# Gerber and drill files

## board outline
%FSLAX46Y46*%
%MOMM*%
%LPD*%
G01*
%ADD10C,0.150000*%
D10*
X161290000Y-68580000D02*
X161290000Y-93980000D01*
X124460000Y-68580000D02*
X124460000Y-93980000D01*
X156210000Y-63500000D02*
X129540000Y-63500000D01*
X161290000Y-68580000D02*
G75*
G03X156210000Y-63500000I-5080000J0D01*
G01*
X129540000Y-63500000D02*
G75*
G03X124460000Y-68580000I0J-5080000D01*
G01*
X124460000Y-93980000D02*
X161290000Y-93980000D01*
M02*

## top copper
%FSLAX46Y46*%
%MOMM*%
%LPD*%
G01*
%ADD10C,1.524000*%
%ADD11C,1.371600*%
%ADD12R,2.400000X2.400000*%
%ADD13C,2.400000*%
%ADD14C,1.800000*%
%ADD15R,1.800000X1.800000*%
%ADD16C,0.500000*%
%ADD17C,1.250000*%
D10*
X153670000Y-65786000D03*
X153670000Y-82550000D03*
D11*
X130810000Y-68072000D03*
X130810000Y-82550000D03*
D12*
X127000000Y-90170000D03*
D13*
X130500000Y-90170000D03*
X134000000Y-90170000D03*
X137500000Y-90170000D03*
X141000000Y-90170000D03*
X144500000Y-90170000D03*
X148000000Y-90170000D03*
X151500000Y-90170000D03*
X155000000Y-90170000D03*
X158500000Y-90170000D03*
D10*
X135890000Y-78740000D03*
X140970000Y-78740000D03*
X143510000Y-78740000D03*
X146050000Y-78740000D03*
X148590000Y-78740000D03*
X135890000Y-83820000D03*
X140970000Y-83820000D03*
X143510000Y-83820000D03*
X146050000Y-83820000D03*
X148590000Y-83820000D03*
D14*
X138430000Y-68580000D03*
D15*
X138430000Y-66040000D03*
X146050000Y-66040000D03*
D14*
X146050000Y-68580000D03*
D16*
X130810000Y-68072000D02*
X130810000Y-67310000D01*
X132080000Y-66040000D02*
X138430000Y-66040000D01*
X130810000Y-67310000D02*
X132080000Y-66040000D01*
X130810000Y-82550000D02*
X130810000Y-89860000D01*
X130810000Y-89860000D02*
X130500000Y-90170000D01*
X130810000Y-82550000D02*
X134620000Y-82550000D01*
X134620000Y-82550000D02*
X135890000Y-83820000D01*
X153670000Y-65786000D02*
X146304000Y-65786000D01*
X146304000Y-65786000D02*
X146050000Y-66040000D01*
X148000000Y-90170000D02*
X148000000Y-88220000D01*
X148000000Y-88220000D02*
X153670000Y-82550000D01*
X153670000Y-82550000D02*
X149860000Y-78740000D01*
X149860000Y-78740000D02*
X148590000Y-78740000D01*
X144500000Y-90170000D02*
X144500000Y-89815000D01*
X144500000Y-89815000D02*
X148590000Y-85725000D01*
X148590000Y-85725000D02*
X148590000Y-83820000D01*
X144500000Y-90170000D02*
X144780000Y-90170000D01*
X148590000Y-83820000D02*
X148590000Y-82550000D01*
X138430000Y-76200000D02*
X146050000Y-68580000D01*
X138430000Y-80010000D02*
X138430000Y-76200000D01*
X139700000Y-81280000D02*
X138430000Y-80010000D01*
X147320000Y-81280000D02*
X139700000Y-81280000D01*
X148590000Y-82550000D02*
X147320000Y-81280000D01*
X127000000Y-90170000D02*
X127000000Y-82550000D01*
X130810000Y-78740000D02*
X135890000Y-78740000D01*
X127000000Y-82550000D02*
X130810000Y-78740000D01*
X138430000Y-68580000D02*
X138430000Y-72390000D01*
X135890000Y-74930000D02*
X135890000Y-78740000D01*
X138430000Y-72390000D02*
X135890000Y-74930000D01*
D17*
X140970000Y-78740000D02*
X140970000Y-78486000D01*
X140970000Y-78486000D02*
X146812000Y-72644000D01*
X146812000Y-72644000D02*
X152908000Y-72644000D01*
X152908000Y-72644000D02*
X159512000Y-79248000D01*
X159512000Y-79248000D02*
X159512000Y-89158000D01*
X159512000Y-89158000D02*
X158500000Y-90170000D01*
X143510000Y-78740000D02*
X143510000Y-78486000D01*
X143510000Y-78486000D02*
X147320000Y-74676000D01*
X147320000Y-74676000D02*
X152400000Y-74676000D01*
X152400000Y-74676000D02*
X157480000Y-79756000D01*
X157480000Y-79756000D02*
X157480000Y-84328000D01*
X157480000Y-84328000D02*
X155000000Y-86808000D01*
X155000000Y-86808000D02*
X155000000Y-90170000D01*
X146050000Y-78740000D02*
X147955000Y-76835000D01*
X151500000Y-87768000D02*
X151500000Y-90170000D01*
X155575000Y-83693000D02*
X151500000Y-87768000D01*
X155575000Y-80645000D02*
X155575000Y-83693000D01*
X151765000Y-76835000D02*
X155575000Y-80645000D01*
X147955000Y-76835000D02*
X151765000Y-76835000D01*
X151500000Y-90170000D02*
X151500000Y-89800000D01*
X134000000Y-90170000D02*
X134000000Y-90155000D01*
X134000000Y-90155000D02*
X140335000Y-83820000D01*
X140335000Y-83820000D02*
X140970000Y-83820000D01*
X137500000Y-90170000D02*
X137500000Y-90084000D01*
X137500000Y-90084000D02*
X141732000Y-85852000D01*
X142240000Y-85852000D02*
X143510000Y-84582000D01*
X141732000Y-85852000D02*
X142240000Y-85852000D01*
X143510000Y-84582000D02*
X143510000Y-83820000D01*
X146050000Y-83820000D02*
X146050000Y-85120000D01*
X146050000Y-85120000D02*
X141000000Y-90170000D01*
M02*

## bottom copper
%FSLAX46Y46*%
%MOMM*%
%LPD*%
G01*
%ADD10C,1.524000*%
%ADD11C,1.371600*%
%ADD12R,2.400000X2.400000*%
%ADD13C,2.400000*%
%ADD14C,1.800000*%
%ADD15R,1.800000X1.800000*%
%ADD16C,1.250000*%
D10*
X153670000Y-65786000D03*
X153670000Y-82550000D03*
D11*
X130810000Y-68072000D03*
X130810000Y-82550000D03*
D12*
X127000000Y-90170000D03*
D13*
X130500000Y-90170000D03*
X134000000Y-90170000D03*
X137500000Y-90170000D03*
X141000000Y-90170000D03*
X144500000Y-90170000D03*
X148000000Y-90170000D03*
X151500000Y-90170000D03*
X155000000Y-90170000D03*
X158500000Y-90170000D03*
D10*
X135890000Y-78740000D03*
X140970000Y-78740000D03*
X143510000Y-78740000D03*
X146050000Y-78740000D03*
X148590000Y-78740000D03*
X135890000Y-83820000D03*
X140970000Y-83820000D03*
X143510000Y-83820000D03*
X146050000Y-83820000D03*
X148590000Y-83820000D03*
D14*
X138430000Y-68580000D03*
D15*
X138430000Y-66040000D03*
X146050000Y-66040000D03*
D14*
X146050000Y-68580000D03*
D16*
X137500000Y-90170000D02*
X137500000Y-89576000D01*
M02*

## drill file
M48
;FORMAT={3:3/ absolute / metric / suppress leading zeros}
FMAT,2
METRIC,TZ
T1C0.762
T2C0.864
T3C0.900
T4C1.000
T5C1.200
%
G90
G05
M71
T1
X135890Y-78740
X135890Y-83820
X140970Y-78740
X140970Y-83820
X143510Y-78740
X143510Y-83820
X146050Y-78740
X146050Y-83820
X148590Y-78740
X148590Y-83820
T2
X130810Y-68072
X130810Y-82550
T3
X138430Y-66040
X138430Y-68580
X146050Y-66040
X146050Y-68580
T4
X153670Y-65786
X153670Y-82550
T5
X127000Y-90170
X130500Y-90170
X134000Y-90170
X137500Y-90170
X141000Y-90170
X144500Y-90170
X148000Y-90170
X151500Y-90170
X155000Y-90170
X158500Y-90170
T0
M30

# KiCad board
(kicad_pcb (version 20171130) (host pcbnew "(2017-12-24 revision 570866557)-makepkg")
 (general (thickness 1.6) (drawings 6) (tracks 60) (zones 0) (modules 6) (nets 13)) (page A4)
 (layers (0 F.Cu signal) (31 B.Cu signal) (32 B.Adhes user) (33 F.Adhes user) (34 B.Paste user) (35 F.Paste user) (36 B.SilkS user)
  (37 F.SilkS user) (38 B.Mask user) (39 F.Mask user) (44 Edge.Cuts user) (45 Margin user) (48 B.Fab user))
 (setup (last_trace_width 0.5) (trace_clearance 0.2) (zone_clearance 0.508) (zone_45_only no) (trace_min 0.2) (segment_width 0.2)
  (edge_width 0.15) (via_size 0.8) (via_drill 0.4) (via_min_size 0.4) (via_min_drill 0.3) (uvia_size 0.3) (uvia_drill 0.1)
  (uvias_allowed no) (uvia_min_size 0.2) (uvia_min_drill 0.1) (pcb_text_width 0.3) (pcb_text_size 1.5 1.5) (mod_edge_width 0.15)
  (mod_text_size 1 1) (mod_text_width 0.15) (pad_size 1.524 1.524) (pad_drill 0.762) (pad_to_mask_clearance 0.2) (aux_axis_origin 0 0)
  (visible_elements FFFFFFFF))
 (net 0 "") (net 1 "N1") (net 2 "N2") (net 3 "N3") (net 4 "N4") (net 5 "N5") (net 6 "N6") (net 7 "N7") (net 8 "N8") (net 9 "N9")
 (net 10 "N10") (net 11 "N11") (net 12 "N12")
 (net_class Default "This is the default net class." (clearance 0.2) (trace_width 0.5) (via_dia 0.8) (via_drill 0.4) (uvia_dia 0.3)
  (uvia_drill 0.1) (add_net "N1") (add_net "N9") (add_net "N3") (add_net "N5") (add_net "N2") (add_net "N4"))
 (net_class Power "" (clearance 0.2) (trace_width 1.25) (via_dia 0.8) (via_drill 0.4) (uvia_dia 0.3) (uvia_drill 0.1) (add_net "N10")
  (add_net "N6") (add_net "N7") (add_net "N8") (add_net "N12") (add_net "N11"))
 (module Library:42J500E (layer F.Cu) (at 153.67 82.55 270)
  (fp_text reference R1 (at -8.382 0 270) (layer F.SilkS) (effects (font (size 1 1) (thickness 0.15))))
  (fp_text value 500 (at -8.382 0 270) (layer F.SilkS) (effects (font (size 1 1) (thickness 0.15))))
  (pad 1 thru_hole circle (at -16.764 0 270) (size 1.524 1.524) (drill 1) (layers *.Cu *.Mask) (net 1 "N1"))
  (pad 2 thru_hole circle (at 0 0 270) (size 1.524 1.524) (drill 1) (layers *.Cu *.Mask) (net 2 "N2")))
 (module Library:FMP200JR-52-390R (layer F.Cu) (at 130.81 82.55 270)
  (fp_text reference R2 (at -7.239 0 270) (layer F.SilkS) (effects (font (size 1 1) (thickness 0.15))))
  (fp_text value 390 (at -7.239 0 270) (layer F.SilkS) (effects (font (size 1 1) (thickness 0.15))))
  (pad 1 thru_hole circle (at -14.478 0 270) (size 1.3716 1.3716) (drill 0.8636) (layers *.Cu *.Mask) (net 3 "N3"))
  (pad 2 thru_hole circle (at 0 0 270) (size 1.3716 1.3716) (drill 0.8636) (layers *.Cu *.Mask) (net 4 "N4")))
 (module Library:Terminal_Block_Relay (layer F.Cu) (at 127 90.17)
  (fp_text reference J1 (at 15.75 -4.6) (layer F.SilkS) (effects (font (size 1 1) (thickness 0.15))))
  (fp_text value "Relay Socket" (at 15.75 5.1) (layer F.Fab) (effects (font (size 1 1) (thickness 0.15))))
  (pad 1 thru_hole rect (at 0 0) (size 2.4 2.4) (drill 1.2) (layers *.Cu *.Mask) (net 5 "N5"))
  (pad 4 thru_hole circle (at 3.5 0) (size 2.4 2.4) (drill 1.2) (layers *.Cu *.Mask) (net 4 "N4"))
  (pad 5 thru_hole circle (at 7 0) (size 2.4 2.4) (drill 1.2) (layers *.Cu *.Mask) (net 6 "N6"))
  (pad 6 thru_hole circle (at 10.5 0) (size 2.4 2.4) (drill 1.2) (layers *.Cu *.Mask) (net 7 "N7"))
  (pad 7 thru_hole circle (at 14 0) (size 2.4 2.4) (drill 1.2) (layers *.Cu *.Mask) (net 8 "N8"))
  (pad 3 thru_hole circle (at 17.5 0) (size 2.4 2.4) (drill 1.2) (layers *.Cu *.Mask) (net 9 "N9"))
  (pad 2 thru_hole circle (at 21 0) (size 2.4 2.4) (drill 1.2) (layers *.Cu *.Mask) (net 2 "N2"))
  (pad 10 thru_hole circle (at 24.5 0) (size 2.4 2.4) (drill 1.2) (layers *.Cu *.Mask) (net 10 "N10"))
  (pad 9 thru_hole circle (at 28 0) (size 2.4 2.4) (drill 1.2) (layers *.Cu *.Mask) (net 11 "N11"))
  (pad 8 thru_hole circle (at 31.5 0) (size 2.4 2.4) (drill 1.2) (layers *.Cu *.Mask) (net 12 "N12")))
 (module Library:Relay (layer F.Cu) (at 135.89 83.82)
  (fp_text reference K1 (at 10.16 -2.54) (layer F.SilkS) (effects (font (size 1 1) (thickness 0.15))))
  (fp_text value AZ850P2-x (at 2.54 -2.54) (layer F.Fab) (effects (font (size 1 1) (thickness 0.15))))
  (pad 12 thru_hole circle (at 0 -5.08) (size 1.524 1.524) (drill 0.762) (layers *.Cu *.Mask) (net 5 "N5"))
  (pad 10 thru_hole circle (at 5.08 -5.08) (size 1.524 1.524) (drill 0.762) (layers *.Cu *.Mask) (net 12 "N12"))
  (pad 9 thru_hole circle (at 7.62 -5.08) (size 1.524 1.524) (drill 0.762) (layers *.Cu *.Mask) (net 11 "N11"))
  (pad 8 thru_hole circle (at 10.16 -5.08) (size 1.524 1.524) (drill 0.762) (layers *.Cu *.Mask) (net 10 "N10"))
  (pad 7 thru_hole circle (at 12.7 -5.08) (size 1.524 1.524) (drill 0.762) (layers *.Cu *.Mask) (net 2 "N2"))
  (pad 1 thru_hole circle (at 0 0) (size 1.524 1.524) (drill 0.762) (layers *.Cu *.Mask) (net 4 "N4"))
  (pad 3 thru_hole circle (at 5.08 0) (size 1.524 1.524) (drill 0.762) (layers *.Cu *.Mask) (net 6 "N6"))
  (pad 4 thru_hole circle (at 7.62 0) (size 1.524 1.524) (drill 0.762) (layers *.Cu *.Mask) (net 7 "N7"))
  (pad 5 thru_hole circle (at 10.16 0) (size 1.524 1.524) (drill 0.762) (layers *.Cu *.Mask) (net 8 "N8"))
  (pad 6 thru_hole circle (at 12.7 0) (size 1.524 1.524) (drill 0.762) (layers *.Cu *.Mask) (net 9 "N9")))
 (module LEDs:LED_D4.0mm (layer F.Cu) (at 138.43 66.04 270)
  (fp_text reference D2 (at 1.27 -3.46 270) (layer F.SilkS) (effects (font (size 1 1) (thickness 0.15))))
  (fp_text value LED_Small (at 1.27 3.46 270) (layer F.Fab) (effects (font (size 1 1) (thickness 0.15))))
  (pad 2 thru_hole circle (at 2.54 0 270) (size 1.8 1.8) (drill 0.9) (layers *.Cu *.Mask) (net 5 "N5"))
  (pad 1 thru_hole rect (at 0 0 270) (size 1.8 1.8) (drill 0.9) (layers *.Cu *.Mask) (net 3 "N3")))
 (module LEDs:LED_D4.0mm (layer F.Cu) (at 146.05 66.04 270)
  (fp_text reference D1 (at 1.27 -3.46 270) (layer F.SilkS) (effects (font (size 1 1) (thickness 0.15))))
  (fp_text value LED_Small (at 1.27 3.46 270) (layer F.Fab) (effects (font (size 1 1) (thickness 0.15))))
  (pad 1 thru_hole rect (at 0 0 270) (size 1.8 1.8) (drill 0.9) (layers *.Cu *.Mask) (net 1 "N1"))
  (pad 2 thru_hole circle (at 2.54 0 270) (size 1.8 1.8) (drill 0.9) (layers *.Cu *.Mask) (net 9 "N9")))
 (gr_line (start 161.29 68.58) (end 161.29 93.98) (angle 90) (layer Edge.Cuts) (width 0.15))
 (gr_line (start 124.46 68.58) (end 124.46 93.98) (angle 90) (layer Edge.Cuts) (width 0.15))
 (gr_line (start 156.21 63.5) (end 129.54 63.5) (angle 90) (layer Edge.Cuts) (width 0.15))
 (gr_arc (start 156.21 68.58) (end 156.21 63.5) (angle 90) (layer Edge.Cuts) (width 0.15))
 (gr_arc (start 129.54 68.58) (end 124.46 68.58) (angle 90) (layer Edge.Cuts) (width 0.15))
 (gr_line (start 124.46 93.98) (end 161.29 93.98) (angle 90) (layer Edge.Cuts) (width 0.15))
 (segment (start 130.81 68.072) (end 130.81 67.31) (width 0.5) (layer F.Cu) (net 3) (status 400000))
 (segment (start 132.08 66.04) (end 138.43 66.04) (width 0.5) (layer F.Cu) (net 3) (status 800000))
 (segment (start 130.81 67.31) (end 132.08 66.04) (width 0.5) (layer F.Cu) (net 3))
 (segment (start 130.81 82.55) (end 130.81 89.86) (width 0.5) (layer F.Cu) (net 4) (status C00000))
 (segment (start 130.81 89.86) (end 130.5 90.17) (width 0.5) (layer F.Cu) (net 4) (status C00000))
 (segment (start 130.81 82.55) (end 134.62 82.55) (width 0.5) (layer F.Cu) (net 4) (status 400000))
 (segment (start 134.62 82.55) (end 135.89 83.82) (width 0.5) (layer F.Cu) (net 4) (status 800000))
 (segment (start 153.67 65.786) (end 146.304 65.786) (width 0.5) (layer F.Cu) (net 1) (status C00000))
 (segment (start 146.304 65.786) (end 146.05 66.04) (width 0.5) (layer F.Cu) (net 1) (status C00000))
 (segment (start 148 90.17) (end 148 88.22) (width 0.5) (layer F.Cu) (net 2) (status 400000))
 (segment (start 148 88.22) (end 153.67 82.55) (width 0.5) (layer F.Cu) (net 2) (status 800000))
 (segment (start 153.67 82.55) (end 149.86 78.74) (width 0.5) (layer F.Cu) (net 2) (status 400000))
 (segment (start 149.86 78.74) (end 148.59 78.74) (width 0.5) (layer F.Cu) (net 2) (status 800000))
 (segment (start 144.5 90.17) (end 144.5 89.815) (width 0.5) (layer F.Cu) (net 9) (status C00000))
 (segment (start 144.5 89.815) (end 148.59 85.725) (width 0.5) (layer F.Cu) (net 9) (status 400000))
 (segment (start 148.59 85.725) (end 148.59 83.82) (width 0.5) (layer F.Cu) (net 9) (status 800000))
 (segment (start 144.5 90.17) (end 144.78 90.17) (width 0.5) (layer F.Cu) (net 9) (status C00000))
 (segment (start 148.59 83.82) (end 148.59 82.55) (width 0.5) (layer F.Cu) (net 9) (status 400000))
 (segment (start 138.43 76.2) (end 146.05 68.58) (width 0.5) (layer F.Cu) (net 9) (status 800000))
 (segment (start 138.43 80.01) (end 138.43 76.2) (width 0.5) (layer F.Cu) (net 9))
 (segment (start 139.7 81.28) (end 138.43 80.01) (width 0.5) (layer F.Cu) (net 9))
 (segment (start 147.32 81.28) (end 139.7 81.28) (width 0.5) (layer F.Cu) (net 9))
 (segment (start 148.59 82.55) (end 147.32 81.28) (width 0.5) (layer F.Cu) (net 9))
 (segment (start 127 90.17) (end 127 82.55) (width 0.5) (layer F.Cu) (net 5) (status 400000))
 (segment (start 130.81 78.74) (end 135.89 78.74) (width 0.5) (layer F.Cu) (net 5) (status 800000))
 (segment (start 127 82.55) (end 130.81 78.74) (width 0.5) (layer F.Cu) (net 5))
 (segment (start 138.43 68.58) (end 138.43 72.39) (width 0.5) (layer F.Cu) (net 5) (status 400000))
 (segment (start 135.89 74.93) (end 135.89 78.74) (width 0.5) (layer F.Cu) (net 5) (status 800000))
 (segment (start 138.43 72.39) (end 135.89 74.93) (width 0.5) (layer F.Cu) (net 5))
 (segment (start 140.97 78.74) (end 140.97 78.486) (width 1.25) (layer F.Cu) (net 12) (status C00000))
 (segment (start 140.97 78.486) (end 146.812 72.644) (width 1.25) (layer F.Cu) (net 12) (status 400000))
 (segment (start 146.812 72.644) (end 152.908 72.644) (width 1.25) (layer F.Cu) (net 12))
 (segment (start 152.908 72.644) (end 159.512 79.248) (width 1.25) (layer F.Cu) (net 12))
 (segment (start 159.512 79.248) (end 159.512 89.158) (width 1.25) (layer F.Cu) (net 12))
 (segment (start 159.512 89.158) (end 158.5 90.17) (width 1.25) (layer F.Cu) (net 12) (status 800000))
 (segment (start 143.51 78.74) (end 143.51 78.486) (width 1.25) (layer F.Cu) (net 11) (status C00000))
 (segment (start 143.51 78.486) (end 147.32 74.676) (width 1.25) (layer F.Cu) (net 11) (status 400000))
 (segment (start 147.32 74.676) (end 152.4 74.676) (width 1.25) (layer F.Cu) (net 11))
 (segment (start 152.4 74.676) (end 157.48 79.756) (width 1.25) (layer F.Cu) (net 11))
 (segment (start 157.48 79.756) (end 157.48 84.328) (width 1.25) (layer F.Cu) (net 11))
 (segment (start 157.48 84.328) (end 155 86.808) (width 1.25) (layer F.Cu) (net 11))
 (segment (start 155 86.808) (end 155 90.17) (width 1.25) (layer F.Cu) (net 11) (status 800000))
 (segment (start 146.05 78.74) (end 147.955 76.835) (width 1.25) (layer F.Cu) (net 10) (status 400000))
 (segment (start 151.5 87.768) (end 151.5 90.17) (width 1.25) (layer F.Cu) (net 10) (status 800000))
 (segment (start 155.575 83.693) (end 151.5 87.768) (width 1.25) (layer F.Cu) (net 10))
 (segment (start 155.575 80.645) (end 155.575 83.693) (width 1.25) (layer F.Cu) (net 10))
 (segment (start 151.765 76.835) (end 155.575 80.645) (width 1.25) (layer F.Cu) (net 10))
 (segment (start 147.955 76.835) (end 151.765 76.835) (width 1.25) (layer F.Cu) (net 10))
 (segment (start 151.5 90.17) (end 151.5 89.8) (width 1.25) (layer F.Cu) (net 10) (status C00000))
 (segment (start 134 90.17) (end 134 90.155) (width 1.25) (layer F.Cu) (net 6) (status C00000))
 (segment (start 134 90.155) (end 140.335 83.82) (width 1.25) (layer F.Cu) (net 6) (status C00000))
 (segment (start 140.335 83.82) (end 140.97 83.82) (width 1.25) (layer F.Cu) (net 6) (status C00000))
 (segment (start 137.5 90.17) (end 137.5 90.084) (width 1.25) (layer F.Cu) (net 7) (status C00000))
 (segment (start 137.5 90.084) (end 141.732 85.852) (width 1.25) (layer F.Cu) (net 7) (status 400000))
 (segment (start 142.24 85.852) (end 143.51 84.582) (width 1.25) (layer F.Cu) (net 7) (status 800000))
 (segment (start 141.732 85.852) (end 142.24 85.852) (width 1.25) (layer F.Cu) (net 7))
 (segment (start 143.51 84.582) (end 143.51 83.82) (width 1.25) (layer F.Cu) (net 7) (status C00000))
 (segment (start 137.5 90.17) (end 137.5 89.576) (width 1.25) (layer B.Cu) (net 7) (status C00000))
 (segment (start 146.05 83.82) (end 146.05 85.12) (width 1.25) (layer F.Cu) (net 8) (status 400000))
 (segment (start 146.05 85.12) (end 141 90.17) (width 1.25) (layer F.Cu) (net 8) (status 800000)))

